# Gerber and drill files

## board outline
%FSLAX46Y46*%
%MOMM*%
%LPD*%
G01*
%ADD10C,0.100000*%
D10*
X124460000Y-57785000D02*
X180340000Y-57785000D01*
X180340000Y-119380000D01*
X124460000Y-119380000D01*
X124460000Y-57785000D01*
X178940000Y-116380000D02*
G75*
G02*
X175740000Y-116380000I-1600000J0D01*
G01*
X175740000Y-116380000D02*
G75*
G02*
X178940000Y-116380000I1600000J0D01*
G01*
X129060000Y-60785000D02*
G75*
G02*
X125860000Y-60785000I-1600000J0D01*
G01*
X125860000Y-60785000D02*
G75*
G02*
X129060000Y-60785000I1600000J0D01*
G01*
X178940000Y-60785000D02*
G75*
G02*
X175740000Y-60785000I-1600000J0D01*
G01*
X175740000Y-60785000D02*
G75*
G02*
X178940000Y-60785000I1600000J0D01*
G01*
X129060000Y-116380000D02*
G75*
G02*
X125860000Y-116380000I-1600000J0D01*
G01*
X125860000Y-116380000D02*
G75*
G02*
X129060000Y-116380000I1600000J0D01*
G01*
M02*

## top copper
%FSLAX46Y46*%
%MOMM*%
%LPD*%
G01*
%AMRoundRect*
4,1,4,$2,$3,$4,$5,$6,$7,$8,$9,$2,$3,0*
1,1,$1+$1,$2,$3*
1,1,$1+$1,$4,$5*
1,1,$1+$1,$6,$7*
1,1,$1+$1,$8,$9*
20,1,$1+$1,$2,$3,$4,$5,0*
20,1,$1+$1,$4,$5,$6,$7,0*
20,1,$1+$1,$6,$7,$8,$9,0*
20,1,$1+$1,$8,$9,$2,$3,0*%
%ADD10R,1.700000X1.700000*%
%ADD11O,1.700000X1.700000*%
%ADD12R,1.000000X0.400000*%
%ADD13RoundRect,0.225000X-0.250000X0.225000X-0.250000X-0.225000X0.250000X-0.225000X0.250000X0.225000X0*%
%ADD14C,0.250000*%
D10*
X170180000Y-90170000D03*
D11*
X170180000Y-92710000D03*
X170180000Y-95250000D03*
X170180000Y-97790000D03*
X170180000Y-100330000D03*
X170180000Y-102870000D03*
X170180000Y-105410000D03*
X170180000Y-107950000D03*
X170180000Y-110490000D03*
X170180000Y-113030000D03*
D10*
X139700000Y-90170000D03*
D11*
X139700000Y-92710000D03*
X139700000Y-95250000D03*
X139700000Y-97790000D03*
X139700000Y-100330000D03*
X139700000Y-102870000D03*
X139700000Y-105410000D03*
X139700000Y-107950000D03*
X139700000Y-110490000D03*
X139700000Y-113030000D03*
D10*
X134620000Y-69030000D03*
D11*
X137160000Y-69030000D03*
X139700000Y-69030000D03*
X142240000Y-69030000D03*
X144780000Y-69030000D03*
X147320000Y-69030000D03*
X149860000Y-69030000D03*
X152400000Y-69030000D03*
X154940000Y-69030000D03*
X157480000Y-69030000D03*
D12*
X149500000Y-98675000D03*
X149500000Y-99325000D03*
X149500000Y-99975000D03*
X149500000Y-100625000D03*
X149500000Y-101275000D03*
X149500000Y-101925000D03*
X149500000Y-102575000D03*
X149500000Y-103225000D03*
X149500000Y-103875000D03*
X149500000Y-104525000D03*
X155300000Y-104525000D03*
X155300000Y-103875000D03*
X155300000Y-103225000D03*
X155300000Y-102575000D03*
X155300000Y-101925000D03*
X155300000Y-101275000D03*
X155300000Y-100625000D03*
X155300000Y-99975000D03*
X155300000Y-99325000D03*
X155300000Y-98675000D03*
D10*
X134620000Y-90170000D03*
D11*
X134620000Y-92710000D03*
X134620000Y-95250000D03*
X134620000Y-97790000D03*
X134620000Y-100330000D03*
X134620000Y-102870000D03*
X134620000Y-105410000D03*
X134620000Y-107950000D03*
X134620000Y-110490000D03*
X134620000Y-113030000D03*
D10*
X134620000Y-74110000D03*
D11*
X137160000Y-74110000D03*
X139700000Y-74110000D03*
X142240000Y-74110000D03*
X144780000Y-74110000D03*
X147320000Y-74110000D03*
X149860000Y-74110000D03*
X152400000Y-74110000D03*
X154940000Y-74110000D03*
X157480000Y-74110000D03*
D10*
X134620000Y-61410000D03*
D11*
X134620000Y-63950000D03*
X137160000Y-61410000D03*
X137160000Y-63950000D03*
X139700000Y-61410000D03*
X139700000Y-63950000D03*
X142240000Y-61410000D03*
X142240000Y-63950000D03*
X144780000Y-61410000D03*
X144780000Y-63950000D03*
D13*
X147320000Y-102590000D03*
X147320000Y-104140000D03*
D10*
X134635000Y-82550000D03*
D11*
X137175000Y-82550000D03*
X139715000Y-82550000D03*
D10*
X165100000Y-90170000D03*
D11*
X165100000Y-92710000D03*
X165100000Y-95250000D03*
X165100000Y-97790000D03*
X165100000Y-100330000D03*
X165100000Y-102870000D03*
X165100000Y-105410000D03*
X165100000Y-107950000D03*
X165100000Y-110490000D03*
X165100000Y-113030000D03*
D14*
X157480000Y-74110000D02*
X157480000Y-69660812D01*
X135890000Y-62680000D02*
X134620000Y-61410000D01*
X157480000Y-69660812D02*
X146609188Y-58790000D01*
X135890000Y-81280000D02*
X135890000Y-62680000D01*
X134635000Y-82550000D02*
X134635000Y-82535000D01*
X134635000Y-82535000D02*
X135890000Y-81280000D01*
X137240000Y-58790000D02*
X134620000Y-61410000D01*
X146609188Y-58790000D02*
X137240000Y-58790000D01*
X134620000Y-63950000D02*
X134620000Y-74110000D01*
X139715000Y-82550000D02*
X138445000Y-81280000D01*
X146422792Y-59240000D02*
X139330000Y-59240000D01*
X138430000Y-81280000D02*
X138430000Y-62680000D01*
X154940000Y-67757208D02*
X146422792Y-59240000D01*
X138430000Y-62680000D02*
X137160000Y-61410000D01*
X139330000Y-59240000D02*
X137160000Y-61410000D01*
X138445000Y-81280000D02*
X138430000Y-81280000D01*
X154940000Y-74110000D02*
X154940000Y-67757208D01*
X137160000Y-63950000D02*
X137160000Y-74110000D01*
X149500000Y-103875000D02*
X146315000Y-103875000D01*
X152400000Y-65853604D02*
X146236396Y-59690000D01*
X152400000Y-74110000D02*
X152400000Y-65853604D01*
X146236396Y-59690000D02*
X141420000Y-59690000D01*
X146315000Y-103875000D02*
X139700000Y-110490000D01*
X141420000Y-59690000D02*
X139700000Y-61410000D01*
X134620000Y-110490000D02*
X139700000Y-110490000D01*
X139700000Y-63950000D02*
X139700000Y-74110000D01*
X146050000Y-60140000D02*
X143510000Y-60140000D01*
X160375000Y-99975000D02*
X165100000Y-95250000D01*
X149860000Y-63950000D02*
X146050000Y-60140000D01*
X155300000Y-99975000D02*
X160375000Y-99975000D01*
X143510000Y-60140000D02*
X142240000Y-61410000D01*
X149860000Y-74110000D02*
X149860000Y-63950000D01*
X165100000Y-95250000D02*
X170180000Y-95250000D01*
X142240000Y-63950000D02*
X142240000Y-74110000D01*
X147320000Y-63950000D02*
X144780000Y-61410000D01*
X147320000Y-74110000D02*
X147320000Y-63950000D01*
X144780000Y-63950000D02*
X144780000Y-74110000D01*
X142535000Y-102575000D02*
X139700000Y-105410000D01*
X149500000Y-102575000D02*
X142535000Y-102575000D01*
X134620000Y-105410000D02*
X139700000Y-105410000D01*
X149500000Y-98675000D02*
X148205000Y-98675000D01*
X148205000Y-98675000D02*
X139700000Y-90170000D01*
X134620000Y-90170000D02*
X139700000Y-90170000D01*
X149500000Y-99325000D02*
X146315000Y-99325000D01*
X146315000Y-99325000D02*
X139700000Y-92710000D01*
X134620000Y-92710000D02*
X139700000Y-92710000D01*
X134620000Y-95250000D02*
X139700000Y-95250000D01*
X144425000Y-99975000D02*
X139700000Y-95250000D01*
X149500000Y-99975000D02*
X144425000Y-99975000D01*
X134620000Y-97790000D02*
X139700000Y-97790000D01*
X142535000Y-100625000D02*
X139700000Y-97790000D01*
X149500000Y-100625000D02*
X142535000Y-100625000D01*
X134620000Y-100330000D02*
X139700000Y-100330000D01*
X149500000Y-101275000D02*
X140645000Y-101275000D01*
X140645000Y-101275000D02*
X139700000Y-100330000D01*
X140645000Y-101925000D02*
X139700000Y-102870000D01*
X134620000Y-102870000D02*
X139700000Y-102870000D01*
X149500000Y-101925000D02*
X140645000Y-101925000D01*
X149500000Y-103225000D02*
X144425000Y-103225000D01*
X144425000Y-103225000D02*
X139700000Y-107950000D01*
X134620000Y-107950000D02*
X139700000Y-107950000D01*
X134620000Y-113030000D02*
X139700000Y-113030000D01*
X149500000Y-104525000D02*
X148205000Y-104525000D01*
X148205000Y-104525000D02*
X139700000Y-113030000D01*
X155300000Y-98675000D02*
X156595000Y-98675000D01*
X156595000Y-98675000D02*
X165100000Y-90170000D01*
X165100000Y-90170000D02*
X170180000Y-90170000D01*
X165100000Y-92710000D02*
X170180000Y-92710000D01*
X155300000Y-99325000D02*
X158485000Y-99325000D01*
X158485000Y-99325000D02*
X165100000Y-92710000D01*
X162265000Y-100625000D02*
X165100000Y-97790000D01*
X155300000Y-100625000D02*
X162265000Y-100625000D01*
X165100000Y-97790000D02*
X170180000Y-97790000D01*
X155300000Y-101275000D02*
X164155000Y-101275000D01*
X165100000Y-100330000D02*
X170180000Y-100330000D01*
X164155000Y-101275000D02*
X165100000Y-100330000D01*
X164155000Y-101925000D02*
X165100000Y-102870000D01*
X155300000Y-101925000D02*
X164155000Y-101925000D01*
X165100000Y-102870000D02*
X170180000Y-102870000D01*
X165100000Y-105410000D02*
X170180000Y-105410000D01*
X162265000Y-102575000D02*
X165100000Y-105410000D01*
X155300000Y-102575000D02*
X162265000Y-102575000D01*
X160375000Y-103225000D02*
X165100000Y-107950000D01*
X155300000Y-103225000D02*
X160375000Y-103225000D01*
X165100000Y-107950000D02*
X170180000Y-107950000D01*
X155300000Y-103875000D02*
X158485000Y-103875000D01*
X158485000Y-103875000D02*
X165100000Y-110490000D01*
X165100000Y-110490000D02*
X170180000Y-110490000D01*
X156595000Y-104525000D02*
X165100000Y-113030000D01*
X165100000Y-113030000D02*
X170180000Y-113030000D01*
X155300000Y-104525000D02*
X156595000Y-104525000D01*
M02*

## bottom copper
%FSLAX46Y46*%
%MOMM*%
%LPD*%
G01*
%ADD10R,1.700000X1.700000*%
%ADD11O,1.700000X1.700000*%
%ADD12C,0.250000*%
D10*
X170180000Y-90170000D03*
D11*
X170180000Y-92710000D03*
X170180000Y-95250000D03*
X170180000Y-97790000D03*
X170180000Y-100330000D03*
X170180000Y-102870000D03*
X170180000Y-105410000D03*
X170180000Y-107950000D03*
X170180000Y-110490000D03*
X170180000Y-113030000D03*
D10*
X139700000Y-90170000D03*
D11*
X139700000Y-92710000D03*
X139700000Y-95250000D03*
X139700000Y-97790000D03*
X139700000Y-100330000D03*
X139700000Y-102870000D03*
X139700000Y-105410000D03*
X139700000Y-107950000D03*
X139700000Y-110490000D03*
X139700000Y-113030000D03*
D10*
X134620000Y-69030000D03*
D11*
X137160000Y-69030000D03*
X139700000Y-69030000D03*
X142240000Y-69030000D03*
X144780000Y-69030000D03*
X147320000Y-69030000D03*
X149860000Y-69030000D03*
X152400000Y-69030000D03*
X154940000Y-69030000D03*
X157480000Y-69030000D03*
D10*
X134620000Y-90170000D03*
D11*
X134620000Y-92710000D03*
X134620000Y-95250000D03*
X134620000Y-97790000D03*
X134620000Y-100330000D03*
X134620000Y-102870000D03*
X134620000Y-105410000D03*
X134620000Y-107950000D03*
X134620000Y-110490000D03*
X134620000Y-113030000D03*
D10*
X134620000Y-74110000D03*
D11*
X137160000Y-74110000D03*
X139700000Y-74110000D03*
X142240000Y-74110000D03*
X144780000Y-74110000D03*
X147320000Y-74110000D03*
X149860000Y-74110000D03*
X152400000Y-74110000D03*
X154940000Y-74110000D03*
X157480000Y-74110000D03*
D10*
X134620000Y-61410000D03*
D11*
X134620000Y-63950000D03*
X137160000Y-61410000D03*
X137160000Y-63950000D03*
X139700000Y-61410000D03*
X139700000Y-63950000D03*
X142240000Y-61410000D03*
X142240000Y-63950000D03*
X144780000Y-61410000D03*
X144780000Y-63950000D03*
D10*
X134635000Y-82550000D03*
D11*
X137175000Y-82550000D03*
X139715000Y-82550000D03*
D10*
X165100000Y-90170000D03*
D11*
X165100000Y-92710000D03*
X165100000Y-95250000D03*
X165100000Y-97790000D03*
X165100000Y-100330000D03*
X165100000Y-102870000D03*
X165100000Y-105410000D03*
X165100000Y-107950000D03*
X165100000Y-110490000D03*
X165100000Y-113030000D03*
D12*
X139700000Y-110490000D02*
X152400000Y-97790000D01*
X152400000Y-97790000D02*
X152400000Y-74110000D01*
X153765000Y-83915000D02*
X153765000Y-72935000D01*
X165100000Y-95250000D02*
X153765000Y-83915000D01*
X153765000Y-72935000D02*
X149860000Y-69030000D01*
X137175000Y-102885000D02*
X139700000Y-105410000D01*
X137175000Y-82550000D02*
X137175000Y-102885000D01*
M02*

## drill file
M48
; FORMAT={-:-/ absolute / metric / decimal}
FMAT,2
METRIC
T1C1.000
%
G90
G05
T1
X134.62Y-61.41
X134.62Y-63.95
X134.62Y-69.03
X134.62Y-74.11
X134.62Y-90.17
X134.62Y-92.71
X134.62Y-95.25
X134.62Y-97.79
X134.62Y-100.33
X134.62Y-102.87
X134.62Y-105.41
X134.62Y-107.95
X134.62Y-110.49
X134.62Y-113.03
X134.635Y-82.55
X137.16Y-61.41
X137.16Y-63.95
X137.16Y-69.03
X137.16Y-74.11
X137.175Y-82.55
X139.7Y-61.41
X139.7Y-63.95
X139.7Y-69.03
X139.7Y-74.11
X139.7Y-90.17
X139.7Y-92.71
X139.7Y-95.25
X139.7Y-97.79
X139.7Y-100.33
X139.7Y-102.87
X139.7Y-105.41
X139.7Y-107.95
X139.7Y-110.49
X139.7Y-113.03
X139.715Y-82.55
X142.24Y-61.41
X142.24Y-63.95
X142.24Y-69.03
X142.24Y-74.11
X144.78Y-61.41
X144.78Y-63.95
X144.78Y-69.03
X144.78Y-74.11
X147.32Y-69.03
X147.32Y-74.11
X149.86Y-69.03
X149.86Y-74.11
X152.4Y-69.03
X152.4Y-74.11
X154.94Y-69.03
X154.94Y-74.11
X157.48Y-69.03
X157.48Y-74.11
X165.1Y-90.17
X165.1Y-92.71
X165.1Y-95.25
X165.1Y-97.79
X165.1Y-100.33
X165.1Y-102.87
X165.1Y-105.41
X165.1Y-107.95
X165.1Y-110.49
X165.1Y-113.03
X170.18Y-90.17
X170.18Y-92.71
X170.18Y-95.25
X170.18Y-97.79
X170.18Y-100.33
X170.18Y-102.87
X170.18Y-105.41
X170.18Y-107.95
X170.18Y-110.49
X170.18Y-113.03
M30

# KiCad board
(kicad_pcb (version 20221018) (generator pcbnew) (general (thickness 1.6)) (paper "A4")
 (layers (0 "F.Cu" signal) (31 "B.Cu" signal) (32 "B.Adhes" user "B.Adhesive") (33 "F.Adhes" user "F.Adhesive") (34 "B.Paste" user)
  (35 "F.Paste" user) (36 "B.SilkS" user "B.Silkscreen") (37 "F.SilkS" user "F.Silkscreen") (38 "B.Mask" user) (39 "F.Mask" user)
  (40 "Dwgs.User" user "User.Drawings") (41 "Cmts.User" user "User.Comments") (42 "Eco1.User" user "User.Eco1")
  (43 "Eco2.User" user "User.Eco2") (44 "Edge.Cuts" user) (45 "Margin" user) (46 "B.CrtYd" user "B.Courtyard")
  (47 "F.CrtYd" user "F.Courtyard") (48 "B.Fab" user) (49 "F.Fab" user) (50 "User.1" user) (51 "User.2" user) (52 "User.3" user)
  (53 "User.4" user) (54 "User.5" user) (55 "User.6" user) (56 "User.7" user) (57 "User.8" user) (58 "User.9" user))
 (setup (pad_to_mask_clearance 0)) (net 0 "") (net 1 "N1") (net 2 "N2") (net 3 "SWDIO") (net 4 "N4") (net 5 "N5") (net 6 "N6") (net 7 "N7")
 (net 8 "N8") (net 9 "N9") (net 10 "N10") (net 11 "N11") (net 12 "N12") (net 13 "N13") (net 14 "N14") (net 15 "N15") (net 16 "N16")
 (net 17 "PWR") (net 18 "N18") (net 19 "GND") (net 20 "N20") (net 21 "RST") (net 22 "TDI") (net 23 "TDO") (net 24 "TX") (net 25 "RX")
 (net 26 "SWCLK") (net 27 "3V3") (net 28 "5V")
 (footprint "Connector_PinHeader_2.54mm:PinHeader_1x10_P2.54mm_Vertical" (layer "F.Cu") (at 170.18 90.17)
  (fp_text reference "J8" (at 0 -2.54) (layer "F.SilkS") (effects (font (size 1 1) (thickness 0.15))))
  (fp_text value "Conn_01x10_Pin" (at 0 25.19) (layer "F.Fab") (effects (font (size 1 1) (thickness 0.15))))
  (pad "1" thru_hole rect (at 0 0) (size 1.7 1.7) (drill 1) (layers "*.Cu" "*.Mask") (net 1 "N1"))
  (pad "2" thru_hole oval (at 0 2.54) (size 1.7 1.7) (drill 1) (layers "*.Cu" "*.Mask") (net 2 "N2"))
  (pad "3" thru_hole oval (at 0 5.08) (size 1.7 1.7) (drill 1) (layers "*.Cu" "*.Mask") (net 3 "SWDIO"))
  (pad "4" thru_hole oval (at 0 7.62) (size 1.7 1.7) (drill 1) (layers "*.Cu" "*.Mask") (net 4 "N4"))
  (pad "5" thru_hole oval (at 0 10.16) (size 1.7 1.7) (drill 1) (layers "*.Cu" "*.Mask") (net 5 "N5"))
  (pad "6" thru_hole oval (at 0 12.7) (size 1.7 1.7) (drill 1) (layers "*.Cu" "*.Mask") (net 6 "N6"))
  (pad "7" thru_hole oval (at 0 15.24) (size 1.7 1.7) (drill 1) (layers "*.Cu" "*.Mask") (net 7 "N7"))
  (pad "8" thru_hole oval (at 0 17.78) (size 1.7 1.7) (drill 1) (layers "*.Cu" "*.Mask") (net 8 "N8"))
  (pad "9" thru_hole oval (at 0 20.32) (size 1.7 1.7) (drill 1) (layers "*.Cu" "*.Mask") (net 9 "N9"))
  (pad "10" thru_hole oval (at 0 22.86) (size 1.7 1.7) (drill 1) (layers "*.Cu" "*.Mask") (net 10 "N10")))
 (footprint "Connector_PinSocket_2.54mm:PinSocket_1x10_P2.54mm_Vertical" (layer "F.Cu") (at 139.7 90.17)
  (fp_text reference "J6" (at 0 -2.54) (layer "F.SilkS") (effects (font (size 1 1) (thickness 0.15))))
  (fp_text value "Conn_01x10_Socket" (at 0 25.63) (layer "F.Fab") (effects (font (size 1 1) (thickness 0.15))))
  (pad "1" thru_hole rect (at 0 0) (size 1.7 1.7) (drill 1) (layers "*.Cu" "*.Mask") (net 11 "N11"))
  (pad "2" thru_hole oval (at 0 2.54) (size 1.7 1.7) (drill 1) (layers "*.Cu" "*.Mask") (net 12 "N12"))
  (pad "3" thru_hole oval (at 0 5.08) (size 1.7 1.7) (drill 1) (layers "*.Cu" "*.Mask") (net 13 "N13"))
  (pad "4" thru_hole oval (at 0 7.62) (size 1.7 1.7) (drill 1) (layers "*.Cu" "*.Mask") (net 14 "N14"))
  (pad "5" thru_hole oval (at 0 10.16) (size 1.7 1.7) (drill 1) (layers "*.Cu" "*.Mask") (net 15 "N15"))
  (pad "6" thru_hole oval (at 0 12.7) (size 1.7 1.7) (drill 1) (layers "*.Cu" "*.Mask") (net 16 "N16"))
  (pad "7" thru_hole oval (at 0 15.24) (size 1.7 1.7) (drill 1) (layers "*.Cu" "*.Mask") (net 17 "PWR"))
  (pad "8" thru_hole oval (at 0 17.78) (size 1.7 1.7) (drill 1) (layers "*.Cu" "*.Mask") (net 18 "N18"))
  (pad "9" thru_hole oval (at 0 20.32) (size 1.7 1.7) (drill 1) (layers "*.Cu" "*.Mask") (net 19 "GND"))
  (pad "10" thru_hole oval (at 0 22.86) (size 1.7 1.7) (drill 1) (layers "*.Cu" "*.Mask") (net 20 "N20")))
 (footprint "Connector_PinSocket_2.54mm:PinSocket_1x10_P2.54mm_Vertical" (layer "F.Cu") (at 134.62 69.03 90)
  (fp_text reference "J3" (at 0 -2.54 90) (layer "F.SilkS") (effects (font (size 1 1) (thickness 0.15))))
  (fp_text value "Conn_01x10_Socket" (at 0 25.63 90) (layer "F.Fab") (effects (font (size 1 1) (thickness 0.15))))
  (pad "1" thru_hole rect (at 0 0 90) (size 1.7 1.7) (drill 1) (layers "*.Cu" "*.Mask") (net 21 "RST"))
  (pad "2" thru_hole oval (at 0 2.54 90) (size 1.7 1.7) (drill 1) (layers "*.Cu" "*.Mask") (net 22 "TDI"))
  (pad "3" thru_hole oval (at 0 5.08 90) (size 1.7 1.7) (drill 1) (layers "*.Cu" "*.Mask") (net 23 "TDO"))
  (pad "4" thru_hole oval (at 0 7.62 90) (size 1.7 1.7) (drill 1) (layers "*.Cu" "*.Mask") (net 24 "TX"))
  (pad "5" thru_hole oval (at 0 10.16 90) (size 1.7 1.7) (drill 1) (layers "*.Cu" "*.Mask") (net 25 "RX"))
  (pad "6" thru_hole oval (at 0 12.7 90) (size 1.7 1.7) (drill 1) (layers "*.Cu" "*.Mask") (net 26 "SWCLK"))
  (pad "7" thru_hole oval (at 0 15.24 90) (size 1.7 1.7) (drill 1) (layers "*.Cu" "*.Mask") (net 3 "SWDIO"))
  (pad "8" thru_hole oval (at 0 17.78 90) (size 1.7 1.7) (drill 1) (layers "*.Cu" "*.Mask") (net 19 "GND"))
  (pad "9" thru_hole oval (at 0 20.32 90) (size 1.7 1.7) (drill 1) (layers "*.Cu" "*.Mask") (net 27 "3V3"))
  (pad "10" thru_hole oval (at 0 22.86 90) (size 1.7 1.7) (drill 1) (layers "*.Cu" "*.Mask") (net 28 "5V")))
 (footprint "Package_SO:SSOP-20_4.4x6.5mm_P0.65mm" (layer "F.Cu") (at 152.4 101.6)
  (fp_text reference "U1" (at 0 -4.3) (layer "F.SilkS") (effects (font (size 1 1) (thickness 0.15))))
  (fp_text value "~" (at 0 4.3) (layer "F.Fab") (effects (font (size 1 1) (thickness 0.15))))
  (pad "1" smd rect (at -2.9 -2.925) (size 1 0.4) (layers "F.Cu" "F.Paste" "F.Mask") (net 11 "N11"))
  (pad "2" smd rect (at -2.9 -2.275) (size 1 0.4) (layers "F.Cu" "F.Paste" "F.Mask") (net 12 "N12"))
  (pad "3" smd rect (at -2.9 -1.625) (size 1 0.4) (layers "F.Cu" "F.Paste" "F.Mask") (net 13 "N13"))
  (pad "4" smd rect (at -2.9 -0.975) (size 1 0.4) (layers "F.Cu" "F.Paste" "F.Mask") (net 14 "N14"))
  (pad "5" smd rect (at -2.9 -0.325) (size 1 0.4) (layers "F.Cu" "F.Paste" "F.Mask") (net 15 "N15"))
  (pad "6" smd rect (at -2.9 0.325) (size 1 0.4) (layers "F.Cu" "F.Paste" "F.Mask") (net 16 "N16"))
  (pad "7" smd rect (at -2.9 0.975) (size 1 0.4) (layers "F.Cu" "F.Paste" "F.Mask") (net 17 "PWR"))
  (pad "8" smd rect (at -2.9 1.625) (size 1 0.4) (layers "F.Cu" "F.Paste" "F.Mask") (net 18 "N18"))
  (pad "9" smd rect (at -2.9 2.275) (size 1 0.4) (layers "F.Cu" "F.Paste" "F.Mask") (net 19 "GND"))
  (pad "10" smd rect (at -2.9 2.925) (size 1 0.4) (layers "F.Cu" "F.Paste" "F.Mask") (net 20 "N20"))
  (pad "11" smd rect (at 2.9 2.925) (size 1 0.4) (layers "F.Cu" "F.Paste" "F.Mask") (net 10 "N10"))
  (pad "12" smd rect (at 2.9 2.275) (size 1 0.4) (layers "F.Cu" "F.Paste" "F.Mask") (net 9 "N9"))
  (pad "13" smd rect (at 2.9 1.625) (size 1 0.4) (layers "F.Cu" "F.Paste" "F.Mask") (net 8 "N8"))
  (pad "14" smd rect (at 2.9 0.975) (size 1 0.4) (layers "F.Cu" "F.Paste" "F.Mask") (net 7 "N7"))
  (pad "15" smd rect (at 2.9 0.325) (size 1 0.4) (layers "F.Cu" "F.Paste" "F.Mask") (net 6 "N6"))
  (pad "16" smd rect (at 2.9 -0.325) (size 1 0.4) (layers "F.Cu" "F.Paste" "F.Mask") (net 5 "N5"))
  (pad "17" smd rect (at 2.9 -0.975) (size 1 0.4) (layers "F.Cu" "F.Paste" "F.Mask") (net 4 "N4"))
  (pad "18" smd rect (at 2.9 -1.625) (size 1 0.4) (layers "F.Cu" "F.Paste" "F.Mask") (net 3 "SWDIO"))
  (pad "19" smd rect (at 2.9 -2.275) (size 1 0.4) (layers "F.Cu" "F.Paste" "F.Mask") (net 2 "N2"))
  (pad "20" smd rect (at 2.9 -2.925) (size 1 0.4) (layers "F.Cu" "F.Paste" "F.Mask") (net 1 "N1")))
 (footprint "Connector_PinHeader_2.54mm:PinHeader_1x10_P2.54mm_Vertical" (layer "F.Cu") (at 134.62 90.17)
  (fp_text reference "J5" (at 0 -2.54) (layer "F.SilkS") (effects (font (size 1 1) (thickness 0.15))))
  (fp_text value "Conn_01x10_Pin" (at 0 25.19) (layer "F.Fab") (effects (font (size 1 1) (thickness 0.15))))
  (pad "1" thru_hole rect (at 0 0) (size 1.7 1.7) (drill 1) (layers "*.Cu" "*.Mask") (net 11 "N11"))
  (pad "2" thru_hole oval (at 0 2.54) (size 1.7 1.7) (drill 1) (layers "*.Cu" "*.Mask") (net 12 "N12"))
  (pad "3" thru_hole oval (at 0 5.08) (size 1.7 1.7) (drill 1) (layers "*.Cu" "*.Mask") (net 13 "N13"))
  (pad "4" thru_hole oval (at 0 7.62) (size 1.7 1.7) (drill 1) (layers "*.Cu" "*.Mask") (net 14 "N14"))
  (pad "5" thru_hole oval (at 0 10.16) (size 1.7 1.7) (drill 1) (layers "*.Cu" "*.Mask") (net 15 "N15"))
  (pad "6" thru_hole oval (at 0 12.7) (size 1.7 1.7) (drill 1) (layers "*.Cu" "*.Mask") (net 16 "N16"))
  (pad "7" thru_hole oval (at 0 15.24) (size 1.7 1.7) (drill 1) (layers "*.Cu" "*.Mask") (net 17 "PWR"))
  (pad "8" thru_hole oval (at 0 17.78) (size 1.7 1.7) (drill 1) (layers "*.Cu" "*.Mask") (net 18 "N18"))
  (pad "9" thru_hole oval (at 0 20.32) (size 1.7 1.7) (drill 1) (layers "*.Cu" "*.Mask") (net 19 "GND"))
  (pad "10" thru_hole oval (at 0 22.86) (size 1.7 1.7) (drill 1) (layers "*.Cu" "*.Mask") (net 20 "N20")))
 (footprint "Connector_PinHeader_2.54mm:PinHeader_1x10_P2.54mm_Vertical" (layer "F.Cu") (at 134.62 74.11 90)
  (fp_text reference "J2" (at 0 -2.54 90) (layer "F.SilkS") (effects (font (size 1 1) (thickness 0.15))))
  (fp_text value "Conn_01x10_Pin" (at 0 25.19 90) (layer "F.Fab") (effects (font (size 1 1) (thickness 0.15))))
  (pad "1" thru_hole rect (at 0 0 90) (size 1.7 1.7) (drill 1) (layers "*.Cu" "*.Mask") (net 21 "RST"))
  (pad "2" thru_hole oval (at 0 2.54 90) (size 1.7 1.7) (drill 1) (layers "*.Cu" "*.Mask") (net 22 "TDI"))
  (pad "3" thru_hole oval (at 0 5.08 90) (size 1.7 1.7) (drill 1) (layers "*.Cu" "*.Mask") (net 23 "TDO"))
  (pad "4" thru_hole oval (at 0 7.62 90) (size 1.7 1.7) (drill 1) (layers "*.Cu" "*.Mask") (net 24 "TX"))
  (pad "5" thru_hole oval (at 0 10.16 90) (size 1.7 1.7) (drill 1) (layers "*.Cu" "*.Mask") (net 25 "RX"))
  (pad "6" thru_hole oval (at 0 12.7 90) (size 1.7 1.7) (drill 1) (layers "*.Cu" "*.Mask") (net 26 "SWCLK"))
  (pad "7" thru_hole oval (at 0 15.24 90) (size 1.7 1.7) (drill 1) (layers "*.Cu" "*.Mask") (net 3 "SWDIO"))
  (pad "8" thru_hole oval (at 0 17.78 90) (size 1.7 1.7) (drill 1) (layers "*.Cu" "*.Mask") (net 19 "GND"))
  (pad "9" thru_hole oval (at 0 20.32 90) (size 1.7 1.7) (drill 1) (layers "*.Cu" "*.Mask") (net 27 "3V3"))
  (pad "10" thru_hole oval (at 0 22.86 90) (size 1.7 1.7) (drill 1) (layers "*.Cu" "*.Mask") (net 28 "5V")))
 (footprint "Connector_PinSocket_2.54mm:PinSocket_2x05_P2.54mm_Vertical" (layer "F.Cu") (at 134.62 61.41 90)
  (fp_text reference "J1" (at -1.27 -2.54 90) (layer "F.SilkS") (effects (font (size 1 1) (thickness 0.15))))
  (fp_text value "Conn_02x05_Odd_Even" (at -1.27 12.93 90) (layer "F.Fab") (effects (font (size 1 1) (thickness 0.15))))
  (pad "1" thru_hole rect (at 0 0 90) (size 1.7 1.7) (drill 1) (layers "*.Cu" "*.Mask") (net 28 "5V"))
  (pad "2" thru_hole oval (at -2.54 0 90) (size 1.7 1.7) (drill 1) (layers "*.Cu" "*.Mask") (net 21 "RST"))
  (pad "3" thru_hole oval (at 0 2.54 90) (size 1.7 1.7) (drill 1) (layers "*.Cu" "*.Mask") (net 27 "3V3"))
  (pad "4" thru_hole oval (at -2.54 2.54 90) (size 1.7 1.7) (drill 1) (layers "*.Cu" "*.Mask") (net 22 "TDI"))
  (pad "5" thru_hole oval (at 0 5.08 90) (size 1.7 1.7) (drill 1) (layers "*.Cu" "*.Mask") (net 19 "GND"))
  (pad "6" thru_hole oval (at -2.54 5.08 90) (size 1.7 1.7) (drill 1) (layers "*.Cu" "*.Mask") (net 23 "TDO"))
  (pad "7" thru_hole oval (at 0 7.62 90) (size 1.7 1.7) (drill 1) (layers "*.Cu" "*.Mask") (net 3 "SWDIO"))
  (pad "8" thru_hole oval (at -2.54 7.62 90) (size 1.7 1.7) (drill 1) (layers "*.Cu" "*.Mask") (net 24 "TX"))
  (pad "9" thru_hole oval (at 0 10.16 90) (size 1.7 1.7) (drill 1) (layers "*.Cu" "*.Mask") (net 26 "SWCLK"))
  (pad "10" thru_hole oval (at -2.54 10.16 90) (size 1.7 1.7) (drill 1) (layers "*.Cu" "*.Mask") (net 25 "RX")))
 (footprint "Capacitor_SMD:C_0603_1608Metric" (layer "F.Cu") (at 147.32 103.365 -90)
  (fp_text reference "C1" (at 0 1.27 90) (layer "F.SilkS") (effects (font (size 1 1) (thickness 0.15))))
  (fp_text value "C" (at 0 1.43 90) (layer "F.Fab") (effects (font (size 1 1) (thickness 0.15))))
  (pad "1" smd roundrect (at -0.775 0 270) (size 0.9 0.95) (layers "F.Cu" "F.Paste" "F.Mask") (roundrect_rratio 0.25) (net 17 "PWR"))
  (pad "2" smd roundrect (at 0.775 0 270) (size 0.9 0.95) (layers "F.Cu" "F.Paste" "F.Mask") (roundrect_rratio 0.25) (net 19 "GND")))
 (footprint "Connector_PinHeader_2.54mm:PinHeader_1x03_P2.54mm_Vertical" (layer "F.Cu") (at 134.635 82.55 90)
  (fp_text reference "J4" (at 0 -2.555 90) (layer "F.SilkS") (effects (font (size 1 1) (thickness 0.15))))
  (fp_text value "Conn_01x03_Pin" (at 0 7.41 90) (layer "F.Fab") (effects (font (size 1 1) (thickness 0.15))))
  (pad "1" thru_hole rect (at 0 0 90) (size 1.7 1.7) (drill 1) (layers "*.Cu" "*.Mask") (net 28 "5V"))
  (pad "2" thru_hole oval (at 0 2.54 90) (size 1.7 1.7) (drill 1) (layers "*.Cu" "*.Mask") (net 17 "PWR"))
  (pad "3" thru_hole oval (at 0 5.08 90) (size 1.7 1.7) (drill 1) (layers "*.Cu" "*.Mask") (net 27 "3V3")))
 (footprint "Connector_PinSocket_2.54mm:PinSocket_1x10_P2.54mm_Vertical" (layer "F.Cu") (at 165.1 90.17)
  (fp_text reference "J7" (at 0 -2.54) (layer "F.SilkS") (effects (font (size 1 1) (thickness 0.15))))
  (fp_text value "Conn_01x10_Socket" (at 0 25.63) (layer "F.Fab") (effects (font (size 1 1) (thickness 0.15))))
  (pad "1" thru_hole rect (at 0 0) (size 1.7 1.7) (drill 1) (layers "*.Cu" "*.Mask") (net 1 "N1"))
  (pad "2" thru_hole oval (at 0 2.54) (size 1.7 1.7) (drill 1) (layers "*.Cu" "*.Mask") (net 2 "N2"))
  (pad "3" thru_hole oval (at 0 5.08) (size 1.7 1.7) (drill 1) (layers "*.Cu" "*.Mask") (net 3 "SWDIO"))
  (pad "4" thru_hole oval (at 0 7.62) (size 1.7 1.7) (drill 1) (layers "*.Cu" "*.Mask") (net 4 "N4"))
  (pad "5" thru_hole oval (at 0 10.16) (size 1.7 1.7) (drill 1) (layers "*.Cu" "*.Mask") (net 5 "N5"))
  (pad "6" thru_hole oval (at 0 12.7) (size 1.7 1.7) (drill 1) (layers "*.Cu" "*.Mask") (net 6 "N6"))
  (pad "7" thru_hole oval (at 0 15.24) (size 1.7 1.7) (drill 1) (layers "*.Cu" "*.Mask") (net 7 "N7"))
  (pad "8" thru_hole oval (at 0 17.78) (size 1.7 1.7) (drill 1) (layers "*.Cu" "*.Mask") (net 8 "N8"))
  (pad "9" thru_hole oval (at 0 20.32) (size 1.7 1.7) (drill 1) (layers "*.Cu" "*.Mask") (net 9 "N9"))
  (pad "10" thru_hole oval (at 0 22.86) (size 1.7 1.7) (drill 1) (layers "*.Cu" "*.Mask") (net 10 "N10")))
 (gr_rect (start 124.46 57.785) (end 180.34 119.38) (stroke (width 0.1) (type default)) (fill none) (layer "Edge.Cuts"))
 (gr_circle (center 177.34 116.38) (end 175.74 116.38) (stroke (width 0.1) (type default)) (fill none) (layer "Edge.Cuts"))
 (gr_circle (center 127.46 60.785) (end 129.06 60.785) (stroke (width 0.1) (type default)) (fill none) (layer "Edge.Cuts"))
 (gr_circle (center 177.34 60.785) (end 177.34 62.385) (stroke (width 0.1) (type default)) (fill none) (layer "Edge.Cuts"))
 (gr_circle (center 127.46 116.38) (end 127.46 114.78) (stroke (width 0.1) (type default)) (fill none) (layer "Edge.Cuts"))
 (segment (start 157.48 74.11) (end 157.48 69.660812) (width 0.25) (layer "F.Cu") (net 28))
 (segment (start 135.89 62.68) (end 134.62 61.41) (width 0.25) (layer "F.Cu") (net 28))
 (segment (start 157.48 69.660812) (end 146.609188 58.79) (width 0.25) (layer "F.Cu") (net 28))
 (segment (start 135.89 81.28) (end 135.89 62.68) (width 0.25) (layer "F.Cu") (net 28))
 (segment (start 134.635 82.55) (end 134.635 82.535) (width 0.25) (layer "F.Cu") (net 28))
 (segment (start 134.635 82.535) (end 135.89 81.28) (width 0.25) (layer "F.Cu") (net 28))
 (segment (start 137.24 58.79) (end 134.62 61.41) (width 0.25) (layer "F.Cu") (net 28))
 (segment (start 146.609188 58.79) (end 137.24 58.79) (width 0.25) (layer "F.Cu") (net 28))
 (segment (start 134.62 63.95) (end 134.62 74.11) (width 0.25) (layer "F.Cu") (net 21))
 (segment (start 139.715 82.55) (end 138.445 81.28) (width 0.25) (layer "F.Cu") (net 27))
 (segment (start 146.422792 59.24) (end 139.33 59.24) (width 0.25) (layer "F.Cu") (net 27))
 (segment (start 138.43 81.28) (end 138.43 62.68) (width 0.25) (layer "F.Cu") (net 27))
 (segment (start 154.94 67.757208) (end 146.422792 59.24) (width 0.25) (layer "F.Cu") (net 27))
 (segment (start 138.43 62.68) (end 137.16 61.41) (width 0.25) (layer "F.Cu") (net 27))
 (segment (start 139.33 59.24) (end 137.16 61.41) (width 0.25) (layer "F.Cu") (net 27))
 (segment (start 138.445 81.28) (end 138.43 81.28) (width 0.25) (layer "F.Cu") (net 27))
 (segment (start 154.94 74.11) (end 154.94 67.757208) (width 0.25) (layer "F.Cu") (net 27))
 (segment (start 137.16 63.95) (end 137.16 74.11) (width 0.25) (layer "F.Cu") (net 22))
 (segment (start 149.5 103.875) (end 146.315 103.875) (width 0.25) (layer "F.Cu") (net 19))
 (segment (start 152.4 65.853604) (end 146.236396 59.69) (width 0.25) (layer "F.Cu") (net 19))
 (segment (start 152.4 74.11) (end 152.4 65.853604) (width 0.25) (layer "F.Cu") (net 19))
 (segment (start 146.236396 59.69) (end 141.42 59.69) (width 0.25) (layer "F.Cu") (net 19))
 (segment (start 146.315 103.875) (end 139.7 110.49) (width 0.25) (layer "F.Cu") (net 19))
 (segment (start 141.42 59.69) (end 139.7 61.41) (width 0.25) (layer "F.Cu") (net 19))
 (segment (start 134.62 110.49) (end 139.7 110.49) (width 0.25) (layer "F.Cu") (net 19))
 (segment (start 139.7 110.49) (end 152.4 97.79) (width 0.25) (layer "B.Cu") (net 19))
 (segment (start 152.4 97.79) (end 152.4 74.11) (width 0.25) (layer "B.Cu") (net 19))
 (segment (start 139.7 63.95) (end 139.7 74.11) (width 0.25) (layer "F.Cu") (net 23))
 (segment (start 146.05 60.14) (end 143.51 60.14) (width 0.25) (layer "F.Cu") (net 3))
 (segment (start 160.375 99.975) (end 165.1 95.25) (width 0.25) (layer "F.Cu") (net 3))
 (segment (start 149.86 63.95) (end 146.05 60.14) (width 0.25) (layer "F.Cu") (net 3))
 (segment (start 155.3 99.975) (end 160.375 99.975) (width 0.25) (layer "F.Cu") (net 3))
 (segment (start 143.51 60.14) (end 142.24 61.41) (width 0.25) (layer "F.Cu") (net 3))
 (segment (start 149.86 74.11) (end 149.86 63.95) (width 0.25) (layer "F.Cu") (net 3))
 (segment (start 165.1 95.25) (end 170.18 95.25) (width 0.25) (layer "F.Cu") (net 3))
 (segment (start 153.765 83.915) (end 153.765 72.935) (width 0.25) (layer "B.Cu") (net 3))
 (segment (start 165.1 95.25) (end 153.765 83.915) (width 0.25) (layer "B.Cu") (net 3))
 (segment (start 153.765 72.935) (end 149.86 69.03) (width 0.25) (layer "B.Cu") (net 3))
 (segment (start 142.24 63.95) (end 142.24 74.11) (width 0.25) (layer "F.Cu") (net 24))
 (segment (start 147.32 63.95) (end 144.78 61.41) (width 0.25) (layer "F.Cu") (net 26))
 (segment (start 147.32 74.11) (end 147.32 63.95) (width 0.25) (layer "F.Cu") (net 26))
 (segment (start 144.78 63.95) (end 144.78 74.11) (width 0.25) (layer "F.Cu") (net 25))
 (segment (start 142.535 102.575) (end 139.7 105.41) (width 0.25) (layer "F.Cu") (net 17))
 (segment (start 149.5 102.575) (end 142.535 102.575) (width 0.25) (layer "F.Cu") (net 17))
 (segment (start 134.62 105.41) (end 139.7 105.41) (width 0.25) (layer "F.Cu") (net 17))
 (segment (start 137.175 102.885) (end 139.7 105.41) (width 0.25) (layer "B.Cu") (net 17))
 (segment (start 137.175 82.55) (end 137.175 102.885) (width 0.25) (layer "B.Cu") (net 17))
 (segment (start 149.5 98.675) (end 148.205 98.675) (width 0.25) (layer "F.Cu") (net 11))
 (segment (start 148.205 98.675) (end 139.7 90.17) (width 0.25) (layer "F.Cu") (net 11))
 (segment (start 134.62 90.17) (end 139.7 90.17) (width 0.25) (layer "F.Cu") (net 11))
 (segment (start 149.5 99.325) (end 146.315 99.325) (width 0.25) (layer "F.Cu") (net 12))
 (segment (start 146.315 99.325) (end 139.7 92.71) (width 0.25) (layer "F.Cu") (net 12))
 (segment (start 134.62 92.71) (end 139.7 92.71) (width 0.25) (layer "F.Cu") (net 12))
 (segment (start 134.62 95.25) (end 139.7 95.25) (width 0.25) (layer "F.Cu") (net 13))
 (segment (start 144.425 99.975) (end 139.7 95.25) (width 0.25) (layer "F.Cu") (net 13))
 (segment (start 149.5 99.975) (end 144.425 99.975) (width 0.25) (layer "F.Cu") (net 13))
 (segment (start 134.62 97.79) (end 139.7 97.79) (width 0.25) (layer "F.Cu") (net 14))
 (segment (start 142.535 100.625) (end 139.7 97.79) (width 0.25) (layer "F.Cu") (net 14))
 (segment (start 149.5 100.625) (end 142.535 100.625) (width 0.25) (layer "F.Cu") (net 14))
 (segment (start 134.62 100.33) (end 139.7 100.33) (width 0.25) (layer "F.Cu") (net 15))
 (segment (start 149.5 101.275) (end 140.645 101.275) (width 0.25) (layer "F.Cu") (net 15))
 (segment (start 140.645 101.275) (end 139.7 100.33) (width 0.25) (layer "F.Cu") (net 15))
 (segment (start 140.645 101.925) (end 139.7 102.87) (width 0.25) (layer "F.Cu") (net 16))
 (segment (start 134.62 102.87) (end 139.7 102.87) (width 0.25) (layer "F.Cu") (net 16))
 (segment (start 149.5 101.925) (end 140.645 101.925) (width 0.25) (layer "F.Cu") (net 16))
 (segment (start 149.5 103.225) (end 144.425 103.225) (width 0.25) (layer "F.Cu") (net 18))
 (segment (start 144.425 103.225) (end 139.7 107.95) (width 0.25) (layer "F.Cu") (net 18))
 (segment (start 134.62 107.95) (end 139.7 107.95) (width 0.25) (layer "F.Cu") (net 18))
 (segment (start 134.62 113.03) (end 139.7 113.03) (width 0.25) (layer "F.Cu") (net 20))
 (segment (start 149.5 104.525) (end 148.205 104.525) (width 0.25) (layer "F.Cu") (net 20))
 (segment (start 148.205 104.525) (end 139.7 113.03) (width 0.25) (layer "F.Cu") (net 20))
 (segment (start 155.3 98.675) (end 156.595 98.675) (width 0.25) (layer "F.Cu") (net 1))
 (segment (start 156.595 98.675) (end 165.1 90.17) (width 0.25) (layer "F.Cu") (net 1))
 (segment (start 165.1 90.17) (end 170.18 90.17) (width 0.25) (layer "F.Cu") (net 1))
 (segment (start 165.1 92.71) (end 170.18 92.71) (width 0.25) (layer "F.Cu") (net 2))
 (segment (start 155.3 99.325) (end 158.485 99.325) (width 0.25) (layer "F.Cu") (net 2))
 (segment (start 158.485 99.325) (end 165.1 92.71) (width 0.25) (layer "F.Cu") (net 2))
 (segment (start 162.265 100.625) (end 165.1 97.79) (width 0.25) (layer "F.Cu") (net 4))
 (segment (start 155.3 100.625) (end 162.265 100.625) (width 0.25) (layer "F.Cu") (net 4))
 (segment (start 165.1 97.79) (end 170.18 97.79) (width 0.25) (layer "F.Cu") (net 4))
 (segment (start 155.3 101.275) (end 164.155 101.275) (width 0.25) (layer "F.Cu") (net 5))
 (segment (start 165.1 100.33) (end 170.18 100.33) (width 0.25) (layer "F.Cu") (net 5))
 (segment (start 164.155 101.275) (end 165.1 100.33) (width 0.25) (layer "F.Cu") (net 5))
 (segment (start 164.155 101.925) (end 165.1 102.87) (width 0.25) (layer "F.Cu") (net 6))
 (segment (start 155.3 101.925) (end 164.155 101.925) (width 0.25) (layer "F.Cu") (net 6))
 (segment (start 165.1 102.87) (end 170.18 102.87) (width 0.25) (layer "F.Cu") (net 6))
 (segment (start 165.1 105.41) (end 170.18 105.41) (width 0.25) (layer "F.Cu") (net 7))
 (segment (start 162.265 102.575) (end 165.1 105.41) (width 0.25) (layer "F.Cu") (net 7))
 (segment (start 155.3 102.575) (end 162.265 102.575) (width 0.25) (layer "F.Cu") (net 7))
 (segment (start 160.375 103.225) (end 165.1 107.95) (width 0.25) (layer "F.Cu") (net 8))
 (segment (start 155.3 103.225) (end 160.375 103.225) (width 0.25) (layer "F.Cu") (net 8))
 (segment (start 165.1 107.95) (end 170.18 107.95) (width 0.25) (layer "F.Cu") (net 8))
 (segment (start 155.3 103.875) (end 158.485 103.875) (width 0.25) (layer "F.Cu") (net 9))
 (segment (start 158.485 103.875) (end 165.1 110.49) (width 0.25) (layer "F.Cu") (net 9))
 (segment (start 165.1 110.49) (end 170.18 110.49) (width 0.25) (layer "F.Cu") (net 9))
 (segment (start 156.595 104.525) (end 165.1 113.03) (width 0.25) (layer "F.Cu") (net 10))
 (segment (start 165.1 113.03) (end 170.18 113.03) (width 0.25) (layer "F.Cu") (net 10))
 (segment (start 155.3 104.525) (end 156.595 104.525) (width 0.25) (layer "F.Cu") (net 10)))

